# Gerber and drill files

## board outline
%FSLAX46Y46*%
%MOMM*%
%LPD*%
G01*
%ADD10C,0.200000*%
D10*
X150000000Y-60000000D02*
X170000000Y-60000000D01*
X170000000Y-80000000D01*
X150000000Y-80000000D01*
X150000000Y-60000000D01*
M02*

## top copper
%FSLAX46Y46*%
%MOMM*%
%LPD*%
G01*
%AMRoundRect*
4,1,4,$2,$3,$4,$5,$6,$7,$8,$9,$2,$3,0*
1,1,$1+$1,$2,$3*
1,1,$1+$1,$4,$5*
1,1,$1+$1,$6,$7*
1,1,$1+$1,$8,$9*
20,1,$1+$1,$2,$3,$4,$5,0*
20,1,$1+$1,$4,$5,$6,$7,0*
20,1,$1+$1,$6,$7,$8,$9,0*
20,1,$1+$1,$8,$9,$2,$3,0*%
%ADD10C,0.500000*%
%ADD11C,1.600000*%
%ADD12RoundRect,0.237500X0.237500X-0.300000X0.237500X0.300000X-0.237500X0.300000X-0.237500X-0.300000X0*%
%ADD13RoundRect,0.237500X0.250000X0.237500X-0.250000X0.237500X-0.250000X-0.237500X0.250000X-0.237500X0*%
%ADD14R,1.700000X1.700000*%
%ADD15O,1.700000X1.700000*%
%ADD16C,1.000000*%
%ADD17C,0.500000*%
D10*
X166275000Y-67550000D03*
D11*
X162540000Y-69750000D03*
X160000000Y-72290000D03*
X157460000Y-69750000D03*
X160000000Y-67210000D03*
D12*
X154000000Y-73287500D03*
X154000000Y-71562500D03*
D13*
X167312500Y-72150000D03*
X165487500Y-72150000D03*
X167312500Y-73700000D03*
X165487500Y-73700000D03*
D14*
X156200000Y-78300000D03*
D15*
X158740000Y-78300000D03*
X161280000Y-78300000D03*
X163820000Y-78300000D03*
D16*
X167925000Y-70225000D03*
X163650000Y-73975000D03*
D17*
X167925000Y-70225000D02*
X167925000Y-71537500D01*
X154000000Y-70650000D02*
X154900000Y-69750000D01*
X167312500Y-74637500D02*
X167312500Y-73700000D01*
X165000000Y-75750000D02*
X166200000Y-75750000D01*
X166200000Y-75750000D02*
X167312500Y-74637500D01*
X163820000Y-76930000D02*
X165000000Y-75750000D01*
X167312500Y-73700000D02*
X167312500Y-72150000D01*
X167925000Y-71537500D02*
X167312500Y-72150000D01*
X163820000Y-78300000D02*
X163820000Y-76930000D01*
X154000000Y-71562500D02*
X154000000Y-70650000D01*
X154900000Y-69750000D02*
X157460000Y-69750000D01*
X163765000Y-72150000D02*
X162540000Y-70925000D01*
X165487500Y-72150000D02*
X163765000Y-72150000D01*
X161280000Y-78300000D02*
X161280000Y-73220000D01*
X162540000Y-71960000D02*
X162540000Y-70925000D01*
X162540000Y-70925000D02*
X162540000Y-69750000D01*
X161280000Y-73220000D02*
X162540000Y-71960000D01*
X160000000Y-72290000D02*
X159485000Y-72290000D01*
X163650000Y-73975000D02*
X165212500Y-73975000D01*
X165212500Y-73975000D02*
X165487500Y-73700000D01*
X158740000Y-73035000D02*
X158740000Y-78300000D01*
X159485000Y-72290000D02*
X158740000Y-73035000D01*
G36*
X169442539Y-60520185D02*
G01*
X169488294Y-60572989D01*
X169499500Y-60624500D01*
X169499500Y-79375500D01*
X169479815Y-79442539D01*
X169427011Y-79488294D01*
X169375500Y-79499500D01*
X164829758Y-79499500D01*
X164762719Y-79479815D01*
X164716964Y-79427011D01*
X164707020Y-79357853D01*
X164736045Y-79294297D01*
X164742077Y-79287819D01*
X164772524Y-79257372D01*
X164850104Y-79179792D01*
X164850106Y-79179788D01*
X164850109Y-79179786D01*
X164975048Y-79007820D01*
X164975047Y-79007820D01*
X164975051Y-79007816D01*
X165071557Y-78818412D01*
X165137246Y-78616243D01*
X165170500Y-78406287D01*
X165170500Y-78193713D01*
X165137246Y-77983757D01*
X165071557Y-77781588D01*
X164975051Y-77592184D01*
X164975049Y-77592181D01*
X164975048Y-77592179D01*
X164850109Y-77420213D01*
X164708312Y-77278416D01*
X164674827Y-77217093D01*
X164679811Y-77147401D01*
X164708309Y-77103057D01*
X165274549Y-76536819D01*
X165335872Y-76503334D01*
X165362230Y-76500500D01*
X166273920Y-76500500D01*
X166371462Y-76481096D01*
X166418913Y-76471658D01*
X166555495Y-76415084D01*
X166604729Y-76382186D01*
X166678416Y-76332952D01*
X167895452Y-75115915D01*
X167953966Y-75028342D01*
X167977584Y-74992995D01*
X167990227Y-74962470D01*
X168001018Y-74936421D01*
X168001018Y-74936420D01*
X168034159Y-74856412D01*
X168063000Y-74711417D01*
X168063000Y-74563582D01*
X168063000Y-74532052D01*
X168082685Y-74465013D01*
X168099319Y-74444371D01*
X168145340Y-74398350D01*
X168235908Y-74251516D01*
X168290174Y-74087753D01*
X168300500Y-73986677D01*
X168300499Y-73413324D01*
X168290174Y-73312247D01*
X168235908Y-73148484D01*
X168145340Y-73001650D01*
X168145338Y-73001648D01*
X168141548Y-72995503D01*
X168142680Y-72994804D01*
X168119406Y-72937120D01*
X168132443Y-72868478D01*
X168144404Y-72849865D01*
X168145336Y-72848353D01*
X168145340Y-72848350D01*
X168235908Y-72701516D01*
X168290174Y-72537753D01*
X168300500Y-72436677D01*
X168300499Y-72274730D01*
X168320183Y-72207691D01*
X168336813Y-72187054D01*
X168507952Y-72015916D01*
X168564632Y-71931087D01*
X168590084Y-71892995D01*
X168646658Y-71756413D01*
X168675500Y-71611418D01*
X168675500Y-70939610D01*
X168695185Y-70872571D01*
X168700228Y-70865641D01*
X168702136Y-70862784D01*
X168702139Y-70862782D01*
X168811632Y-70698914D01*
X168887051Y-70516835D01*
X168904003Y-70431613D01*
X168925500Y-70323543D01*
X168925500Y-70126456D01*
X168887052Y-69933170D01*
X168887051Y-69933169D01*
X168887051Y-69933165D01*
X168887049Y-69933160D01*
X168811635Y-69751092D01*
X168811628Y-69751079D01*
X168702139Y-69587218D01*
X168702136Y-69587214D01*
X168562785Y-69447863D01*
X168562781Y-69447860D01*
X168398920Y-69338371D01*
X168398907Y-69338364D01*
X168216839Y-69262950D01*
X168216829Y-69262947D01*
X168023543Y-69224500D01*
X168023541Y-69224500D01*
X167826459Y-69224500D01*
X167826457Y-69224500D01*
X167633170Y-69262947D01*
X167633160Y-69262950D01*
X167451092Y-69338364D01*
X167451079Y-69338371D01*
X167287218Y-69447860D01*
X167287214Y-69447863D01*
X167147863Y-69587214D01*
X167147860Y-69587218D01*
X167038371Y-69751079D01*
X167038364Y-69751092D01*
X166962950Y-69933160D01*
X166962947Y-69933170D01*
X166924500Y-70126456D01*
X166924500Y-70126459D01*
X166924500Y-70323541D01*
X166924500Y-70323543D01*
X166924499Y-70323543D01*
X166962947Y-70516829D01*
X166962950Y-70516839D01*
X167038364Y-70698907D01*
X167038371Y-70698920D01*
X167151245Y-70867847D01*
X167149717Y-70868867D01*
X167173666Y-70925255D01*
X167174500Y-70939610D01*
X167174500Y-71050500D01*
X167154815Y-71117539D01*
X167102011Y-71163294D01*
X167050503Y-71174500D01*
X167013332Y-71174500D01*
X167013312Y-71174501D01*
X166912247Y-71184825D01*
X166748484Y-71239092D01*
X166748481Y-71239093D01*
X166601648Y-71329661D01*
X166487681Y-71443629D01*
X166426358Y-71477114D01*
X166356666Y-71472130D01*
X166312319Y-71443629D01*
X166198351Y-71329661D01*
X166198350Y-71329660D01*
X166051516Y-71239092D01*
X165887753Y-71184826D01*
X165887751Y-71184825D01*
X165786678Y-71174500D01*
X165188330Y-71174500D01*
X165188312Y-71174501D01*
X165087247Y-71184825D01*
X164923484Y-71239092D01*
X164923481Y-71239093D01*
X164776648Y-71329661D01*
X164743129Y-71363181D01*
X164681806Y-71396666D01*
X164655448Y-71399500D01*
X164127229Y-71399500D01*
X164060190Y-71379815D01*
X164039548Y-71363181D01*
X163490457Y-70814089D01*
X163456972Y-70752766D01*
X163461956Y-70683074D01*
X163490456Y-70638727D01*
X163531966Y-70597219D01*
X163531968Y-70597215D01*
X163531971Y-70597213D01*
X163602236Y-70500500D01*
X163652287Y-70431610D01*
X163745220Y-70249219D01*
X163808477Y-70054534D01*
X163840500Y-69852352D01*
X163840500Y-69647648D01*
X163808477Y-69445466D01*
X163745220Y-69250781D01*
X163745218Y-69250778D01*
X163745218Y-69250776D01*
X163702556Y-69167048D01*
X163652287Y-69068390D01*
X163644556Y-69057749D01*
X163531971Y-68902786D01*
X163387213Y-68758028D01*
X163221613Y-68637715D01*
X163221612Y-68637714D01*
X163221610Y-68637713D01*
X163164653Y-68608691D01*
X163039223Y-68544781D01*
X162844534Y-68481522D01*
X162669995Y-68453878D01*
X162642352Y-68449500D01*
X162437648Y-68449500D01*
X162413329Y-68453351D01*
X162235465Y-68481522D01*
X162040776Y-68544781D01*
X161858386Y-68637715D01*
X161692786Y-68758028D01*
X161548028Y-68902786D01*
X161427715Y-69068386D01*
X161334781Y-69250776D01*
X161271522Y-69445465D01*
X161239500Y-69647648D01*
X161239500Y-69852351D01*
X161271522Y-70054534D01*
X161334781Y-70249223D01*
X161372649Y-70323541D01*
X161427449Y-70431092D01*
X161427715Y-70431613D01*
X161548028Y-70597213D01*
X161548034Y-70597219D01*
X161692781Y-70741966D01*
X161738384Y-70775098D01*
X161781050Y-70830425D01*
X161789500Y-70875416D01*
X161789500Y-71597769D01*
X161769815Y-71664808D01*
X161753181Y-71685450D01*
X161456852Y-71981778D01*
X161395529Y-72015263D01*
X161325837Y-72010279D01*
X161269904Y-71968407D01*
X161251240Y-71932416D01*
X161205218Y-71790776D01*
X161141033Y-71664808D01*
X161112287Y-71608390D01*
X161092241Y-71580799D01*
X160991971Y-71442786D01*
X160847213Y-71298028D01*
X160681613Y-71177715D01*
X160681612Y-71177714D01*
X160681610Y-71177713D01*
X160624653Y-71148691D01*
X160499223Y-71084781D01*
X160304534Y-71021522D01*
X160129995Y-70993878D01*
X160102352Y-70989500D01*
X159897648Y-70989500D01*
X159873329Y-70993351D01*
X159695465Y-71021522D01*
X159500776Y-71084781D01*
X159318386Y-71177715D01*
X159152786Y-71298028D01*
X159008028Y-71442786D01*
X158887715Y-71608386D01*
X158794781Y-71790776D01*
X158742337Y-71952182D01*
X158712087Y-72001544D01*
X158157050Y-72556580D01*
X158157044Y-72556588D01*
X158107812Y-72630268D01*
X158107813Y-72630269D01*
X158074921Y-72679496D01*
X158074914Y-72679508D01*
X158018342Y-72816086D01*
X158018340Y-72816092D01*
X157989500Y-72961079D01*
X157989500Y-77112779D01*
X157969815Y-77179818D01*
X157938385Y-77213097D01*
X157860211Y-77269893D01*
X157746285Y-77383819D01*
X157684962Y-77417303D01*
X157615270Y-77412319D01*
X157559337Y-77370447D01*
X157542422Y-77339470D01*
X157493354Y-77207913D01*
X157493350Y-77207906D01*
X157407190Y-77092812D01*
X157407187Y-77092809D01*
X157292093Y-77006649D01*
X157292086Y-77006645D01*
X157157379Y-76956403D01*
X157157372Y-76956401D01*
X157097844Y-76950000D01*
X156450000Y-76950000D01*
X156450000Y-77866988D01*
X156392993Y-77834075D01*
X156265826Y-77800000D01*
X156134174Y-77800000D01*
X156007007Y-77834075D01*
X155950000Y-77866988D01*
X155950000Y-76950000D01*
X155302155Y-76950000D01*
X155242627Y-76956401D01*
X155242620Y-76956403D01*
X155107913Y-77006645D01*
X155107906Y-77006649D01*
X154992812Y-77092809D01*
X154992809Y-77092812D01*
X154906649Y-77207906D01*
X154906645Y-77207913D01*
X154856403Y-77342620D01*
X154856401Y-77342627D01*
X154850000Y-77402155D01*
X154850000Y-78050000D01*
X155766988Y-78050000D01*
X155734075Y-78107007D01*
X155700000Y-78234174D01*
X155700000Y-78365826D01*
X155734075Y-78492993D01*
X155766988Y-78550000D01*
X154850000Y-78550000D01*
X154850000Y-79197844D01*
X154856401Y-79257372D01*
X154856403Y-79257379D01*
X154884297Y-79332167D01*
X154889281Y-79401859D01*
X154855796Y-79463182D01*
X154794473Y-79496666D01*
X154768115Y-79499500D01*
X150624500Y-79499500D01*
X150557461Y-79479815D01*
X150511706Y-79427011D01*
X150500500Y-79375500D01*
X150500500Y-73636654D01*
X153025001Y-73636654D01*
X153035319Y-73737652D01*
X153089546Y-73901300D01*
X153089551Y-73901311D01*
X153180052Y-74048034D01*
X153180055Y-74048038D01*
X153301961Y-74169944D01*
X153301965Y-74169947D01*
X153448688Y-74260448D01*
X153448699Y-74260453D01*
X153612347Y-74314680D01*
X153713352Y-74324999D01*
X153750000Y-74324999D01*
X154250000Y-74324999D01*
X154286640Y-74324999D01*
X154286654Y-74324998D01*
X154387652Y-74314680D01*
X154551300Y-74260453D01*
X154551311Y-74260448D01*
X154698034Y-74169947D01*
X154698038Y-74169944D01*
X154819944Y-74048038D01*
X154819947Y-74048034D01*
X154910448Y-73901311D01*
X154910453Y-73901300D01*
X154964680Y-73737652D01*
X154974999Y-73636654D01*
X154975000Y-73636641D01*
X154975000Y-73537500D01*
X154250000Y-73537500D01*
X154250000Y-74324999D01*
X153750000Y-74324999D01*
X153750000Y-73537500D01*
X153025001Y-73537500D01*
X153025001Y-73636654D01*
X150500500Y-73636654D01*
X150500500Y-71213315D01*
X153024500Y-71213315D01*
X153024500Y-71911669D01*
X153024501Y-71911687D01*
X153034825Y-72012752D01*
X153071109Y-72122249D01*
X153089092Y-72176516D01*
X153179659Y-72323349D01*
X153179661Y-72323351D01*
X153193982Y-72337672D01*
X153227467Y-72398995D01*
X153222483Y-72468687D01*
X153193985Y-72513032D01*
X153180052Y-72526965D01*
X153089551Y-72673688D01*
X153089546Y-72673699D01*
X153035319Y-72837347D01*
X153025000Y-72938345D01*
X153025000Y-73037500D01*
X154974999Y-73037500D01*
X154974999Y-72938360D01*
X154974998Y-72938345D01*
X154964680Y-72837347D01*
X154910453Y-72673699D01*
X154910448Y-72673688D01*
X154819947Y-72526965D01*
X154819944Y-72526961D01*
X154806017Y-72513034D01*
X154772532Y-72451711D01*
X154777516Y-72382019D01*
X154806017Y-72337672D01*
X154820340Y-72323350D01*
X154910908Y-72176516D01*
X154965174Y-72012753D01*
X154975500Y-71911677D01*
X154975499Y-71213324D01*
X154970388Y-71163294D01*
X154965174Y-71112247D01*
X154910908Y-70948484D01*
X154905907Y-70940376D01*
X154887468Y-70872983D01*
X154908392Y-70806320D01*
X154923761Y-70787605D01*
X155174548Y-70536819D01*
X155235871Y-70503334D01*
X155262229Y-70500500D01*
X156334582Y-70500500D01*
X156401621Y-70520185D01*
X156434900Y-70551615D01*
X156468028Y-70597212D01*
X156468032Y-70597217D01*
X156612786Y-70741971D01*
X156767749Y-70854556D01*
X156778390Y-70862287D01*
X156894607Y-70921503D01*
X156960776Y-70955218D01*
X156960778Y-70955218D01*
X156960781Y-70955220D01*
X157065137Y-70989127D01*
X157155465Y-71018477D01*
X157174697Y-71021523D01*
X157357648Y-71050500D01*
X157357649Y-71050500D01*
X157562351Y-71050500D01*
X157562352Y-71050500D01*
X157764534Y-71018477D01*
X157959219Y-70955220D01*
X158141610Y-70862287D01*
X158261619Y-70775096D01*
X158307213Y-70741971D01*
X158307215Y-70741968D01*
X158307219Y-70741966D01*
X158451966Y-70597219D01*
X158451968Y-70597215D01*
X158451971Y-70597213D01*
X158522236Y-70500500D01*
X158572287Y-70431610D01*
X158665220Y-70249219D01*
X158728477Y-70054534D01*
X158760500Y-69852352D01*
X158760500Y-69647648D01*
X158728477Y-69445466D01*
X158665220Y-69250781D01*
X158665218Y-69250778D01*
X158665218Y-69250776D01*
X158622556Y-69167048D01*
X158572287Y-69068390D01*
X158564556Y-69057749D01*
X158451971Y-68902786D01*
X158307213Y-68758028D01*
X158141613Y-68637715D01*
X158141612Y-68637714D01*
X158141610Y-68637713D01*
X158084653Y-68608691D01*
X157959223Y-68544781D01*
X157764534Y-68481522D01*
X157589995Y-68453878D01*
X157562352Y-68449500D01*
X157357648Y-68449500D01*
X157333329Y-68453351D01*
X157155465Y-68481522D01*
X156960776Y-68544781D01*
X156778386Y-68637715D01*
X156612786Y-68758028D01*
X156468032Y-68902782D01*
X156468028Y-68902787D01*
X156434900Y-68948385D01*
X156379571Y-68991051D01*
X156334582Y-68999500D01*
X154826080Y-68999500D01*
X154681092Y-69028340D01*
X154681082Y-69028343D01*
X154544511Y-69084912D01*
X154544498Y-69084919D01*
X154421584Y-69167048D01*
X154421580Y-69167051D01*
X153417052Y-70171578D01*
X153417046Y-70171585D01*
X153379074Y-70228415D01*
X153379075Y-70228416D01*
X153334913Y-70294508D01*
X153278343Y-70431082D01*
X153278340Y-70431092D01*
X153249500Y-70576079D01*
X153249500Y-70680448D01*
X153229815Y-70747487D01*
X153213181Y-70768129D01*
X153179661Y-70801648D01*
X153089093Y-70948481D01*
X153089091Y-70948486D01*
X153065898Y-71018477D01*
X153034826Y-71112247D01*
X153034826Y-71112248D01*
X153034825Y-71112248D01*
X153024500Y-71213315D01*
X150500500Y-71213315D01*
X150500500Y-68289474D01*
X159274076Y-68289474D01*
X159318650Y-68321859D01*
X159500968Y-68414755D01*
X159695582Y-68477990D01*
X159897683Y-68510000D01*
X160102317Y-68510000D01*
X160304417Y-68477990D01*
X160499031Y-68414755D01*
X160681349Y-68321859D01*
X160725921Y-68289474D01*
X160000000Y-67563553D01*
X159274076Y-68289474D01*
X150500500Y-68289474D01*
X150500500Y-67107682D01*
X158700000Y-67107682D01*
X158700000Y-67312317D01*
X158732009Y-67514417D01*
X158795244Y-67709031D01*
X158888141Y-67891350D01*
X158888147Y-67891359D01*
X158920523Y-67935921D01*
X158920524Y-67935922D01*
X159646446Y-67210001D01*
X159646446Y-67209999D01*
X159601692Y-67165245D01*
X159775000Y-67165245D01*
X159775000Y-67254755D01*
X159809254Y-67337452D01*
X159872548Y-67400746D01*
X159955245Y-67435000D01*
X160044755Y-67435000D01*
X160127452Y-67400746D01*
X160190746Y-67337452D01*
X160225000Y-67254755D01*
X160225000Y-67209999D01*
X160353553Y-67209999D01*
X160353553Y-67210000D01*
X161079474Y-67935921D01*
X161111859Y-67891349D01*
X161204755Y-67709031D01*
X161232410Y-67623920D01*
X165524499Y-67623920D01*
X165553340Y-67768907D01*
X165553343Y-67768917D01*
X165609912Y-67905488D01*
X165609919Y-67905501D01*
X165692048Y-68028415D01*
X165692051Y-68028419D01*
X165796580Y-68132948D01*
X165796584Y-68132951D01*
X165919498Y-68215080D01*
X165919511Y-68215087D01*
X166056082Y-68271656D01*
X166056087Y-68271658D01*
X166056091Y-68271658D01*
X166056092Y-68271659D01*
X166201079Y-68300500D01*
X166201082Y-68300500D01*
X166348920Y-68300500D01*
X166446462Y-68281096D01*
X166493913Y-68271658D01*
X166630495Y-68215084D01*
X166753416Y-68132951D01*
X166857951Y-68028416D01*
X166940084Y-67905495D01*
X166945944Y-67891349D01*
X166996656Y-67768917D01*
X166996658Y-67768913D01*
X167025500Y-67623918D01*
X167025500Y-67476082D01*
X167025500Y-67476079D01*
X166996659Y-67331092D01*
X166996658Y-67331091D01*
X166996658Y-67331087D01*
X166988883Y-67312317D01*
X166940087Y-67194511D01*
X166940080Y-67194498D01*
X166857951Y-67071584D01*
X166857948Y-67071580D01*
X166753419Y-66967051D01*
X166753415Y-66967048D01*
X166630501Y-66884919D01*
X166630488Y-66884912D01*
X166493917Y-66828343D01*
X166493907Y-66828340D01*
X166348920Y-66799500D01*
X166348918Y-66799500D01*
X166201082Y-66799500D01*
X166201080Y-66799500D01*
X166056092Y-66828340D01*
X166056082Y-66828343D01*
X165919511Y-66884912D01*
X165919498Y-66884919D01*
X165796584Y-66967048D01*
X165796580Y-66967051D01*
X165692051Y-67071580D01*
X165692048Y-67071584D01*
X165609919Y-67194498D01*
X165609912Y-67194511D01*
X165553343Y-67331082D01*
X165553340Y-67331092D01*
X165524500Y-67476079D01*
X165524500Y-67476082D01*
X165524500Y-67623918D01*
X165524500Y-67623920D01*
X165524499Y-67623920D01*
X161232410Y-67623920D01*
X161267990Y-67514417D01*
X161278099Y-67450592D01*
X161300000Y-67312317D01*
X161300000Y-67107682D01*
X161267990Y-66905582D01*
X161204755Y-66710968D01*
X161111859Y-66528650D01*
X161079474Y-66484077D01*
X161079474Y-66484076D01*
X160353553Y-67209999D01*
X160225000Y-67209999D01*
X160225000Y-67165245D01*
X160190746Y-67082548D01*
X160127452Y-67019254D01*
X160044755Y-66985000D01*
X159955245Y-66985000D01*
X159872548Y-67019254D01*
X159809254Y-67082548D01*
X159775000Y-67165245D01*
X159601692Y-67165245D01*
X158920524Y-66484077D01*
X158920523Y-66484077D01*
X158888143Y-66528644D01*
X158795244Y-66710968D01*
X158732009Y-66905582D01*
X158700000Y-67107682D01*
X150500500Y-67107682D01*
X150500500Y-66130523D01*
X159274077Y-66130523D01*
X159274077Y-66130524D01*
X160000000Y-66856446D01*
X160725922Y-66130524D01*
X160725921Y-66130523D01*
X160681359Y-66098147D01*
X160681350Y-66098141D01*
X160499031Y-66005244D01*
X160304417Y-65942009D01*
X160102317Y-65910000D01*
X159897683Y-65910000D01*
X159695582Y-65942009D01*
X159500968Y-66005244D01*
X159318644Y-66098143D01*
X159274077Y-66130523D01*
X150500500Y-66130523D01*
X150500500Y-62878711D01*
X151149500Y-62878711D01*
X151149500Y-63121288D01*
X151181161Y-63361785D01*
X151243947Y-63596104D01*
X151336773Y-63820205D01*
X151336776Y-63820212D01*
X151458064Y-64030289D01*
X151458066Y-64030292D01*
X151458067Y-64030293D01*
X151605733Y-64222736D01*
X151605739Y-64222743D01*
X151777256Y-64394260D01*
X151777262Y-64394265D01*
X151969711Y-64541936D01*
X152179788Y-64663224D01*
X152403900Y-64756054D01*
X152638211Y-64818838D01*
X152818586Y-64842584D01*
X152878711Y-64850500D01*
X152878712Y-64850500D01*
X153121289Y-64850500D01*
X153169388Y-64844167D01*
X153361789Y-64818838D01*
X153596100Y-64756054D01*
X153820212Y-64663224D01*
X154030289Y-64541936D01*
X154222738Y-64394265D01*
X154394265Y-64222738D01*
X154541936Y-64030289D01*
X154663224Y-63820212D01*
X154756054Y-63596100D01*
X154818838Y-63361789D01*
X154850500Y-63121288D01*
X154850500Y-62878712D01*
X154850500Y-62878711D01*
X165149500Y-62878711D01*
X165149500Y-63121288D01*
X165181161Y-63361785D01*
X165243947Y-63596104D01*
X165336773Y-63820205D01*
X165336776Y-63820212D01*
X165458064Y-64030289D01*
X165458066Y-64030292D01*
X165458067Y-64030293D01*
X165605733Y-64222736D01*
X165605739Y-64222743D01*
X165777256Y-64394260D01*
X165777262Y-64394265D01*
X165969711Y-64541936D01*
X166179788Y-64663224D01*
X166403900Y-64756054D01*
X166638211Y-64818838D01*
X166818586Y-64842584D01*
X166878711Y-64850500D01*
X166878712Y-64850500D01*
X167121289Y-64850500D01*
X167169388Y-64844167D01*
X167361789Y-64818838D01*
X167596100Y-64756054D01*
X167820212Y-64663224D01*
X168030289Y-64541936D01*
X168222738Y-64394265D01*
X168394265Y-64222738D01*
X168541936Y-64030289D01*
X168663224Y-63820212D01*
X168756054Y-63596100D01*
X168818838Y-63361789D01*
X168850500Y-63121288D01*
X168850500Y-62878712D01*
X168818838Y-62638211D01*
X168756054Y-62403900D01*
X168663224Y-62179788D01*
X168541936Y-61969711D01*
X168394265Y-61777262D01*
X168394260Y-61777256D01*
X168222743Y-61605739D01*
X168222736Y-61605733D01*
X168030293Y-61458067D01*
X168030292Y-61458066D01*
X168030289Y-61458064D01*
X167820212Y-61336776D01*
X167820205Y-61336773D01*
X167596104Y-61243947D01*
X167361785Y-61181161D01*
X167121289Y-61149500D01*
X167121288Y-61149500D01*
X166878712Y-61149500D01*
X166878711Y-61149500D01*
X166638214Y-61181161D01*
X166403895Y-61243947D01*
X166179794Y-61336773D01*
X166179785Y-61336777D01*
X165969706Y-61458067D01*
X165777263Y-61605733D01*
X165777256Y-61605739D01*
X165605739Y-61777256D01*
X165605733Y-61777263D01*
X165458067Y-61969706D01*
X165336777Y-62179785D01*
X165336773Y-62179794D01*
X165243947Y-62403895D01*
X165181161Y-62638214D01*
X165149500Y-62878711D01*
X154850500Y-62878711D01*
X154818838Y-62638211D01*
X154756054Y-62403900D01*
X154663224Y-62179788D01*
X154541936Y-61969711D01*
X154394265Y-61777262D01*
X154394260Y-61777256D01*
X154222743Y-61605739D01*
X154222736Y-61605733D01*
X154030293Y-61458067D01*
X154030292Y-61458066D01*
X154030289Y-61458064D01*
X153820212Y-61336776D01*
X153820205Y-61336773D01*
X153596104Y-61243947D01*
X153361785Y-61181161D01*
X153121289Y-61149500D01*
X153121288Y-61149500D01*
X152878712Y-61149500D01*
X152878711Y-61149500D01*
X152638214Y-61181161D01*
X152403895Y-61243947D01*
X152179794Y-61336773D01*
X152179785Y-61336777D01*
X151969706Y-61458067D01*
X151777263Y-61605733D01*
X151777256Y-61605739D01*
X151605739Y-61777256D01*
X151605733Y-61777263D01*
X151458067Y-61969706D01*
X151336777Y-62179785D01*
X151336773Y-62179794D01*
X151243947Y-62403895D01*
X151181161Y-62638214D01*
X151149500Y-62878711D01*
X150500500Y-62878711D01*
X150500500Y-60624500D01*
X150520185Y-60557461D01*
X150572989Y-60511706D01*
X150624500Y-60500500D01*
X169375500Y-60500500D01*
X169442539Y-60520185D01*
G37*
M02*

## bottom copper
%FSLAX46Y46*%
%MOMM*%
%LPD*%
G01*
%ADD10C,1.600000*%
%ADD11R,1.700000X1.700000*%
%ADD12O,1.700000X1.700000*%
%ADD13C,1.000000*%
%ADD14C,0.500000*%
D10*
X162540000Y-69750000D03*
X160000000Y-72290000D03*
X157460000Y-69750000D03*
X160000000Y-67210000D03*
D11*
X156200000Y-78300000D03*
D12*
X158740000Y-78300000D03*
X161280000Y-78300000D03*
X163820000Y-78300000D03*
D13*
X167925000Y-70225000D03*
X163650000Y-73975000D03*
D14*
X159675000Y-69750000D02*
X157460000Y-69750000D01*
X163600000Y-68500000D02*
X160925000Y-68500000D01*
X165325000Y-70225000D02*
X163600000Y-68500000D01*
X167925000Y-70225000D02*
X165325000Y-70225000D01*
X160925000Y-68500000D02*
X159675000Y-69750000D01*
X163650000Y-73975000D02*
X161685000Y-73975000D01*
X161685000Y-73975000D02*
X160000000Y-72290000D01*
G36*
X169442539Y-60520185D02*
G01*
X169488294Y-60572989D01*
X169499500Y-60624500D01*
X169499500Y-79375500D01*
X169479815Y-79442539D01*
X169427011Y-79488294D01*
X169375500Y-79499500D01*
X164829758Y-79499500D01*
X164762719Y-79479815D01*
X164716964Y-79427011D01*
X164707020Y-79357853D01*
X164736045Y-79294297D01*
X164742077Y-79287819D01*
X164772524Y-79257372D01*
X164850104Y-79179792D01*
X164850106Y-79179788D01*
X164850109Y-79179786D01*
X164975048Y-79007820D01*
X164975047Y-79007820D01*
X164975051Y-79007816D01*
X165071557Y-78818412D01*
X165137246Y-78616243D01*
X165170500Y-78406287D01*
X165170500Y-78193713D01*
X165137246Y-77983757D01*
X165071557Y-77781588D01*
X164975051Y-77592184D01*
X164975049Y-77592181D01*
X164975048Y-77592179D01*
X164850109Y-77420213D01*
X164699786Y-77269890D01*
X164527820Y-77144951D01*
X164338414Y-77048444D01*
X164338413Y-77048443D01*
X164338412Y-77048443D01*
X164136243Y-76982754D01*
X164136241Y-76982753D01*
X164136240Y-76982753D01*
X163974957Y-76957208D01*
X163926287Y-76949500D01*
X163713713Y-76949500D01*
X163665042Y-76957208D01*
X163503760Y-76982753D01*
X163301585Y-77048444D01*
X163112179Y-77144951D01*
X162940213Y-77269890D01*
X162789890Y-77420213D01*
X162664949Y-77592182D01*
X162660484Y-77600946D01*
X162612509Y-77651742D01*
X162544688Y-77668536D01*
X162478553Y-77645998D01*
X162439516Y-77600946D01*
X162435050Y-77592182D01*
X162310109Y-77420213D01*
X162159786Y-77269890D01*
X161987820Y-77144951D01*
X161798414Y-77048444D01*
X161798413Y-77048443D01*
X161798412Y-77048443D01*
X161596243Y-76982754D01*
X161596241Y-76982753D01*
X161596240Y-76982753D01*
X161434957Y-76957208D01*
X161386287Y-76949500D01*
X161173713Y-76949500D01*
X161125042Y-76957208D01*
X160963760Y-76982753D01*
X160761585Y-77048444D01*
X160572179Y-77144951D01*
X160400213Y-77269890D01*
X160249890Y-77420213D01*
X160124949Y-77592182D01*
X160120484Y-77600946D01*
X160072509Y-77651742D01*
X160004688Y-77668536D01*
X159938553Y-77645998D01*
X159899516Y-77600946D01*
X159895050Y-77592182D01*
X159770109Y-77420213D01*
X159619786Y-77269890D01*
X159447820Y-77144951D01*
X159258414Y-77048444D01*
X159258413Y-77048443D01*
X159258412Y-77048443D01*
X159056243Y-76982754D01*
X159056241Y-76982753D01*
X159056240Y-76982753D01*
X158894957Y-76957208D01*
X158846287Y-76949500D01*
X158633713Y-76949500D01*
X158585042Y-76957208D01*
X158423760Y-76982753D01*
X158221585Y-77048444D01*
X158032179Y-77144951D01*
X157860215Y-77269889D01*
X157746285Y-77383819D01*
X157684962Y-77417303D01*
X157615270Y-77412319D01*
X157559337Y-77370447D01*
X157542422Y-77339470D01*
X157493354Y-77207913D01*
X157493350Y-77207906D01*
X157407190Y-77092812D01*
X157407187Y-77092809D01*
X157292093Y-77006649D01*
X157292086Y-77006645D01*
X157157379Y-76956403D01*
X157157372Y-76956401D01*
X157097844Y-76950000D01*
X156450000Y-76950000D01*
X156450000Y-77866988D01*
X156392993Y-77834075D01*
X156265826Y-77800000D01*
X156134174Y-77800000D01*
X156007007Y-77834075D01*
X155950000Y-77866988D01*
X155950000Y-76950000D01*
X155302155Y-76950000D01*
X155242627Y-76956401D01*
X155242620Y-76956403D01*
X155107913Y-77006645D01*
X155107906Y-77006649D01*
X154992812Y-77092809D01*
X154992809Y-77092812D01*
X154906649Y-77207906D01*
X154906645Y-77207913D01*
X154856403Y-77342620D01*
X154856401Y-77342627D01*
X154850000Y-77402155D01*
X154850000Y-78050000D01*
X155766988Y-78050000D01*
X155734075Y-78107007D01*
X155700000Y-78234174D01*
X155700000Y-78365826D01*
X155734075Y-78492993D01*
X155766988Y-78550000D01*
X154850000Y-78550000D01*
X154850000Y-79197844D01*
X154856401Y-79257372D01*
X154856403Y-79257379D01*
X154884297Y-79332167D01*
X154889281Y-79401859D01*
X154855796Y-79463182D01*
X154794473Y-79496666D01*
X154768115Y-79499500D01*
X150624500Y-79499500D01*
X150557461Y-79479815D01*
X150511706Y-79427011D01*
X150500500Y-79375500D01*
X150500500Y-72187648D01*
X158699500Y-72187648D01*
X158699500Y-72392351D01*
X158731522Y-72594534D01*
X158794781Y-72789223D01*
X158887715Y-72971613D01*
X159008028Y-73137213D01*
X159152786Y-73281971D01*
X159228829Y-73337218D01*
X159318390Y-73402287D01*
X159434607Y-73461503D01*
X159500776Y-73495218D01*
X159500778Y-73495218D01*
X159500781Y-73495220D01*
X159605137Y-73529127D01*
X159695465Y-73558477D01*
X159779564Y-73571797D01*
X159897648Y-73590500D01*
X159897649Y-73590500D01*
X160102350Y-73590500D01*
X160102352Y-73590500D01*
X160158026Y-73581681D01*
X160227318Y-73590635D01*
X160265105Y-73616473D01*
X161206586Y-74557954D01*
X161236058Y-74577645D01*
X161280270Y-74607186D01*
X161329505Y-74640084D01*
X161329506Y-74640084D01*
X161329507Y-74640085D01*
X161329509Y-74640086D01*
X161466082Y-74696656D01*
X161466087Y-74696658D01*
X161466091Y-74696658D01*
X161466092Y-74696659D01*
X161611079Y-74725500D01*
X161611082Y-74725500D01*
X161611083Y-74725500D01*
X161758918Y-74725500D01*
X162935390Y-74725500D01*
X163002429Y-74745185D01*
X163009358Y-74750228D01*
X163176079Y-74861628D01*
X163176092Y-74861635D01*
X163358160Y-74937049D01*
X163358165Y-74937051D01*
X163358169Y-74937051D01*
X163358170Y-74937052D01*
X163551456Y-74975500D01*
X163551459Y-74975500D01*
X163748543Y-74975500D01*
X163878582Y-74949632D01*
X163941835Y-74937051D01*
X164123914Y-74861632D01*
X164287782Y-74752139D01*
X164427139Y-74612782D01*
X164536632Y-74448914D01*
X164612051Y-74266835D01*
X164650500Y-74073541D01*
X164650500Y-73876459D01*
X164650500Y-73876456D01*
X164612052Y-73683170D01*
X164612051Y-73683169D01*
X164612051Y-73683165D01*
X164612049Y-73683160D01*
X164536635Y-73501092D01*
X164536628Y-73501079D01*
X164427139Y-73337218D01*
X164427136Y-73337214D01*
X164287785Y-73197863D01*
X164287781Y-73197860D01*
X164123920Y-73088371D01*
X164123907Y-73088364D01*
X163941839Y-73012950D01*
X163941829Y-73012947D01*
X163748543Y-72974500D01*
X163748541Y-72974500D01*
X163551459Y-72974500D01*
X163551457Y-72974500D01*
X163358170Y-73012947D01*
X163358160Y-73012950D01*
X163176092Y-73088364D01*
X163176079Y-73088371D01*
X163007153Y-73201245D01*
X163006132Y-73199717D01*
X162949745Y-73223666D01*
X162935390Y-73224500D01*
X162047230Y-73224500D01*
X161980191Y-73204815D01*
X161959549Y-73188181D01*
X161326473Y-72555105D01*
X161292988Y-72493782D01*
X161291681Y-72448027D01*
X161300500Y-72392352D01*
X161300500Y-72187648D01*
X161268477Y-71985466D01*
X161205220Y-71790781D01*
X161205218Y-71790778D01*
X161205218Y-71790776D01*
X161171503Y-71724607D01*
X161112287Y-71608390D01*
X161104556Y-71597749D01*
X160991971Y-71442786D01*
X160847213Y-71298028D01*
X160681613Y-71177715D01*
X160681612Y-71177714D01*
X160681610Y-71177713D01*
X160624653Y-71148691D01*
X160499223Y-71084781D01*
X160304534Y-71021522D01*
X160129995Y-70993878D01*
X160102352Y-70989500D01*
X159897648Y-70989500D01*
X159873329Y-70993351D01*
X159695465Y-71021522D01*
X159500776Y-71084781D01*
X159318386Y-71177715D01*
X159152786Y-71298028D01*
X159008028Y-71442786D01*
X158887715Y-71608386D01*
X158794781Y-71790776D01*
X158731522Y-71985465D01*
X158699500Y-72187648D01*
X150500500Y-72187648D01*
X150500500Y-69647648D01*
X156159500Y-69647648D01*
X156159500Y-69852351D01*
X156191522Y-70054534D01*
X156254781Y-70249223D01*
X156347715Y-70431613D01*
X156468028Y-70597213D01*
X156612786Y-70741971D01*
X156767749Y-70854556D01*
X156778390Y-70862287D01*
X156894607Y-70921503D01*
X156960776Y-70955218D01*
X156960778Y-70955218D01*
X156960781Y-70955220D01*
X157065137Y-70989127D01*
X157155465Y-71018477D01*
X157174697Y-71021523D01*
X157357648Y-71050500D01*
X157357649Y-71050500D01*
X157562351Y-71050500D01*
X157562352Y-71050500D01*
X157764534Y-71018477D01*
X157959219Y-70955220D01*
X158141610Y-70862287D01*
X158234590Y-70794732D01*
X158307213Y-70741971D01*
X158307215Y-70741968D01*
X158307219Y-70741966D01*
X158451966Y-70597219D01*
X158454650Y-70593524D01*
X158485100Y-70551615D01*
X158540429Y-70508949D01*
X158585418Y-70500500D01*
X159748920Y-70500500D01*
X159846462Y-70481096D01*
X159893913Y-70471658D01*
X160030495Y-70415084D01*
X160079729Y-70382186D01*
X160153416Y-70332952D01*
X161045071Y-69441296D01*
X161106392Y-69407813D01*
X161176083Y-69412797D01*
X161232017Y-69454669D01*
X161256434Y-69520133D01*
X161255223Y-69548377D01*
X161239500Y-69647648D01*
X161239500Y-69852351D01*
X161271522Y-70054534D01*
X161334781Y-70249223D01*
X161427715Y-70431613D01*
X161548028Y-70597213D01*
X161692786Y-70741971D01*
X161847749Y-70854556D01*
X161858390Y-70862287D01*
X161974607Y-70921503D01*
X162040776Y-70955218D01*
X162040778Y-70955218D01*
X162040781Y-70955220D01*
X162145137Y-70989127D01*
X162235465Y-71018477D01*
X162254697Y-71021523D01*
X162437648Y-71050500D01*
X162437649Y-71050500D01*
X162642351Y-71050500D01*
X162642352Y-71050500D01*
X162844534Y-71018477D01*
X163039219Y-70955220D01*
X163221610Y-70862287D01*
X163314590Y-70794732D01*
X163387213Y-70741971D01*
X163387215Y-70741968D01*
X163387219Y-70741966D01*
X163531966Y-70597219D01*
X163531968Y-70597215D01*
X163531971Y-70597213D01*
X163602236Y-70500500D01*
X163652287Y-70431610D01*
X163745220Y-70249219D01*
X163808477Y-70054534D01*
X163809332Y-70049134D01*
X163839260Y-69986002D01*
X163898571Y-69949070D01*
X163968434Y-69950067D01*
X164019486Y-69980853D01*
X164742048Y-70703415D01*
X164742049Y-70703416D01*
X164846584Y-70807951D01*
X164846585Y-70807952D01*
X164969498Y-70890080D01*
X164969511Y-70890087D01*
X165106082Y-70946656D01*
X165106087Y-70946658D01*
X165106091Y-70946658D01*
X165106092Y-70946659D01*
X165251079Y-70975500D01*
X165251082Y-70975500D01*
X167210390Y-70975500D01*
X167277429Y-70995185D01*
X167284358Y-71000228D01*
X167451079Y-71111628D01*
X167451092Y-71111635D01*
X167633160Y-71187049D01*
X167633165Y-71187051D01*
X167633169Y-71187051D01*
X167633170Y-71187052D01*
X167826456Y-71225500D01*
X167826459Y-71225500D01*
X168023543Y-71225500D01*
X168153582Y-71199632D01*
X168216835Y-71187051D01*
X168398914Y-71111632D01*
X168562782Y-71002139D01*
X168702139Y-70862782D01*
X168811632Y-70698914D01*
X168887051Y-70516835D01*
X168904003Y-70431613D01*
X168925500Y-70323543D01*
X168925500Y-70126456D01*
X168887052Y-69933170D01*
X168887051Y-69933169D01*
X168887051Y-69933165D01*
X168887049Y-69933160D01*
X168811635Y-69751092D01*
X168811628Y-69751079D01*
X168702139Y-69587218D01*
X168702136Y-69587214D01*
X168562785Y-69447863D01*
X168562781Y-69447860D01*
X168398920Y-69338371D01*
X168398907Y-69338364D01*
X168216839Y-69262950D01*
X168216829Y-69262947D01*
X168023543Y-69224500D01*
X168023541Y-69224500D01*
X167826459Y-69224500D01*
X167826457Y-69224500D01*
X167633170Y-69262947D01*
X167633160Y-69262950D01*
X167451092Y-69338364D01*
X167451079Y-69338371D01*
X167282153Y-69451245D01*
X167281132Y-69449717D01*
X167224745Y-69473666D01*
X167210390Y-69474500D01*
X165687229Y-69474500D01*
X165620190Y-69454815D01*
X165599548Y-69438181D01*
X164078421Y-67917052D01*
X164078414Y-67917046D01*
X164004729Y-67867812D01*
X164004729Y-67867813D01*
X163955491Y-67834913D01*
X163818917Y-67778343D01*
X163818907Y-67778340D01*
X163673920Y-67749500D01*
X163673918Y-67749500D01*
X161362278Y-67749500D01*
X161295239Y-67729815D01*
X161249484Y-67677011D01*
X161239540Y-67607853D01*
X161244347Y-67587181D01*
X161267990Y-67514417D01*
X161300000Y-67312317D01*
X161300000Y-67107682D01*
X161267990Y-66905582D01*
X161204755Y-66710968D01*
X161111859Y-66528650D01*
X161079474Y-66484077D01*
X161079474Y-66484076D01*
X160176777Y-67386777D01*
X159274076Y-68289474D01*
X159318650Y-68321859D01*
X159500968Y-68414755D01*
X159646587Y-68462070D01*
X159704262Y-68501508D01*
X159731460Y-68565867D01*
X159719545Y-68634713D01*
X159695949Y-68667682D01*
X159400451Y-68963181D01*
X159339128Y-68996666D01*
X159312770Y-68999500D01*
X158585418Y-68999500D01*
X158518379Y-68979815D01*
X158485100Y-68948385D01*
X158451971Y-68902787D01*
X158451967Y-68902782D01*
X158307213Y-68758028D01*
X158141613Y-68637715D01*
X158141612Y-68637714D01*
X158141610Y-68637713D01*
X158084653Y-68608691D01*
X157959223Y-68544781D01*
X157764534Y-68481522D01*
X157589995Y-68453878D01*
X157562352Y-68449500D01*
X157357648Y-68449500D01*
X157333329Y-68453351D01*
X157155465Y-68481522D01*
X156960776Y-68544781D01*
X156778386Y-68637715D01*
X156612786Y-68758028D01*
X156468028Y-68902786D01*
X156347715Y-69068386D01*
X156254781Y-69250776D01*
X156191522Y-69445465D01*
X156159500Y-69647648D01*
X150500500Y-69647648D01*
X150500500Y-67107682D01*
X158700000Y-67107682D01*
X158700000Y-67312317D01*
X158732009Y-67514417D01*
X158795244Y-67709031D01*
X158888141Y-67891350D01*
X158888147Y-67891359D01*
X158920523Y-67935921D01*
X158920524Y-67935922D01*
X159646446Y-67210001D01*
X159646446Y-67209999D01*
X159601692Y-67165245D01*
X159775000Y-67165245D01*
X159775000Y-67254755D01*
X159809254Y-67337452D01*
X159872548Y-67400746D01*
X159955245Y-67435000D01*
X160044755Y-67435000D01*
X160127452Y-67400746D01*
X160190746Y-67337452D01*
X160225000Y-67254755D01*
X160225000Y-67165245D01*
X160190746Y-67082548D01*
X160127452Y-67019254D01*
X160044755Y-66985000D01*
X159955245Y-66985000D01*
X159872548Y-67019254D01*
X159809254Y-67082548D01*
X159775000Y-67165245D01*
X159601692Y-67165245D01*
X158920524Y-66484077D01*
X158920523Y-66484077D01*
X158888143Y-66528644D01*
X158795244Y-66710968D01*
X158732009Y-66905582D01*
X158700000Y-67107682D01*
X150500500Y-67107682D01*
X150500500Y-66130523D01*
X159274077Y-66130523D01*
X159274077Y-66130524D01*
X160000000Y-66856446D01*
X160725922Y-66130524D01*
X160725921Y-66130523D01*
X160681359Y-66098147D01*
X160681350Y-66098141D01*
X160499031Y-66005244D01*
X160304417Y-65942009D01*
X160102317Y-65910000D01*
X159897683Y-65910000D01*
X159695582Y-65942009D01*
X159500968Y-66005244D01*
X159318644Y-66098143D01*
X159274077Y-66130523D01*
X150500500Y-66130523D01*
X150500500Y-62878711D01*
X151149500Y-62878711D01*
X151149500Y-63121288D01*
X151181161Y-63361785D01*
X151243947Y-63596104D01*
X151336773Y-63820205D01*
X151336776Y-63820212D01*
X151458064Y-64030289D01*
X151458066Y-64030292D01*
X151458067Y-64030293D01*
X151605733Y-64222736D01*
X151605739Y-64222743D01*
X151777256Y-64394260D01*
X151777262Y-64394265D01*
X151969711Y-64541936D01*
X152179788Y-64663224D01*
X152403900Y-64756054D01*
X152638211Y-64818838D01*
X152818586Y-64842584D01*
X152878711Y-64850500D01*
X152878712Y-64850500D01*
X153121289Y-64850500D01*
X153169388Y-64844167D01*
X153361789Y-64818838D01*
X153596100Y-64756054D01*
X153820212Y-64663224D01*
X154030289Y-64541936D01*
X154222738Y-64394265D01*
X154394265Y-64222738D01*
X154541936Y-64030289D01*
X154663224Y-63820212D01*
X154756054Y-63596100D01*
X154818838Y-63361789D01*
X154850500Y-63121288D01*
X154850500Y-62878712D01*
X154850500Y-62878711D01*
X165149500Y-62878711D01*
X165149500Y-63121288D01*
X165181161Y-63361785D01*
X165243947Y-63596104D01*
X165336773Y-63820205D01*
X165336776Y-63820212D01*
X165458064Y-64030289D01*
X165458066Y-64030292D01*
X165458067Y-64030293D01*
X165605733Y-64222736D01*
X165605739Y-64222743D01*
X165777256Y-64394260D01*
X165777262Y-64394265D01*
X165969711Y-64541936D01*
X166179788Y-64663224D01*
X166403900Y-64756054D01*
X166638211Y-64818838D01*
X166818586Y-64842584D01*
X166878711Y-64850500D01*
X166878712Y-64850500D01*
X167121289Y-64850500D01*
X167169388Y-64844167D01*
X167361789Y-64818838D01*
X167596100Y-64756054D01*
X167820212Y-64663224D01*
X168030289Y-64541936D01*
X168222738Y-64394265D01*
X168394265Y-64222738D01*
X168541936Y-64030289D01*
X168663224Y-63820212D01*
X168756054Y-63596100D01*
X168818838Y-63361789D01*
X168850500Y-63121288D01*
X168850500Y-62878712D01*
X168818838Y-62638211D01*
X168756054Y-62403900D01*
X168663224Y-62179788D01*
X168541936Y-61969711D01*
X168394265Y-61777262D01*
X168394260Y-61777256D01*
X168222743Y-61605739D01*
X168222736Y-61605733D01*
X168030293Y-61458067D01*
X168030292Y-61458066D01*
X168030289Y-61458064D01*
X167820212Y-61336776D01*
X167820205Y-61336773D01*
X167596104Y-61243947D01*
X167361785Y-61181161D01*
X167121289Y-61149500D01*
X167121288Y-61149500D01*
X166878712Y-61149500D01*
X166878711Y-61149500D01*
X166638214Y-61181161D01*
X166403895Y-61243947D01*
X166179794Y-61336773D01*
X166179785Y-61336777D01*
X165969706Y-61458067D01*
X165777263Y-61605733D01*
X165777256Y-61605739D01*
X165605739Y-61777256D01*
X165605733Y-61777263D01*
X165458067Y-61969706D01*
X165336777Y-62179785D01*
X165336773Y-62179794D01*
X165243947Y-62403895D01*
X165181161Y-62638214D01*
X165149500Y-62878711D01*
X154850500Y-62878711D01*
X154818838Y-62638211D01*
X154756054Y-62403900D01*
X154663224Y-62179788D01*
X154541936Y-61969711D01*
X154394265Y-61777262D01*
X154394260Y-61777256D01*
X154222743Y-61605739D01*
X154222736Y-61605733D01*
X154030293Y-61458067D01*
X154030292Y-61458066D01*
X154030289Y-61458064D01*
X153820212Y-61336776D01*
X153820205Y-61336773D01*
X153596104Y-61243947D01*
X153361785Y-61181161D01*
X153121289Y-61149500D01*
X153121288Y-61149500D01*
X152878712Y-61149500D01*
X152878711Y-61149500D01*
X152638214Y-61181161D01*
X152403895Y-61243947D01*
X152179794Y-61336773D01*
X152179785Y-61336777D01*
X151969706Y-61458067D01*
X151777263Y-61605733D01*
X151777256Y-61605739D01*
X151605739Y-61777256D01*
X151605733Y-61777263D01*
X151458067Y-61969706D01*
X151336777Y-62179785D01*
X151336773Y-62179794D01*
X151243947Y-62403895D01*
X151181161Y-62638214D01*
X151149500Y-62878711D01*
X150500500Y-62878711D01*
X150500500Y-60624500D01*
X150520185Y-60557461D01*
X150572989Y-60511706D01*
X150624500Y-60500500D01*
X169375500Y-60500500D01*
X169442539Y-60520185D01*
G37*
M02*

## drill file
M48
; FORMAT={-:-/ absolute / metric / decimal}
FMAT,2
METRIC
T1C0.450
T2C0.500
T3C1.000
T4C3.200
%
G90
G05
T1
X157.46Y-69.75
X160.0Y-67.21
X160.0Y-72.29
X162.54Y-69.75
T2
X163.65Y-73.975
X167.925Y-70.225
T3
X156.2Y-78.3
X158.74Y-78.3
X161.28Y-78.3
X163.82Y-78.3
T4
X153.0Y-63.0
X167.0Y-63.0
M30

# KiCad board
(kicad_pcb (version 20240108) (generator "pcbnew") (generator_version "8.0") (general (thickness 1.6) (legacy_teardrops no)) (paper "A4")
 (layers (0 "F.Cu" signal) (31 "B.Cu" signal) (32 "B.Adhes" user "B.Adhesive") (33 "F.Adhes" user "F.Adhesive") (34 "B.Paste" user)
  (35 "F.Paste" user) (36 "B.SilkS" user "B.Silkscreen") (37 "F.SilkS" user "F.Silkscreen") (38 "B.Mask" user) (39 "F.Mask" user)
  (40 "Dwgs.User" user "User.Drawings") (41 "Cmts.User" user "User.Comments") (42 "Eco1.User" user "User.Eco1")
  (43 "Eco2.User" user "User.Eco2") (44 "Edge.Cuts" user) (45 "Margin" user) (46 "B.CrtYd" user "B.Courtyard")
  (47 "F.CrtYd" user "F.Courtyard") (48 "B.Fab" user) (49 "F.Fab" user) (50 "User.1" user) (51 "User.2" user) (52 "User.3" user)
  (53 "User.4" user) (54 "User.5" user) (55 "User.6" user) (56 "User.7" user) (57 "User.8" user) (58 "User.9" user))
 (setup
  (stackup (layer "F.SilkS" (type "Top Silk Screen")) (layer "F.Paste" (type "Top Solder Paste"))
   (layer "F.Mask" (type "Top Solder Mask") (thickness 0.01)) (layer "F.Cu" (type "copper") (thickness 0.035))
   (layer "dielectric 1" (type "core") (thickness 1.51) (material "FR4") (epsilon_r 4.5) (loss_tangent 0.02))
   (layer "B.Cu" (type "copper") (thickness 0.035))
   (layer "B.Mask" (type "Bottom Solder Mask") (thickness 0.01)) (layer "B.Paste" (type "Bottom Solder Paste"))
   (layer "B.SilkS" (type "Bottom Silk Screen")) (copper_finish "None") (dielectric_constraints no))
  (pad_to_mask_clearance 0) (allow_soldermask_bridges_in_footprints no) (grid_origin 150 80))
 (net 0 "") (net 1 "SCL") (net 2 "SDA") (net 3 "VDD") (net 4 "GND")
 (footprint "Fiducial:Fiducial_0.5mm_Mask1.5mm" (layer "F.Cu") (at 166.275 67.55)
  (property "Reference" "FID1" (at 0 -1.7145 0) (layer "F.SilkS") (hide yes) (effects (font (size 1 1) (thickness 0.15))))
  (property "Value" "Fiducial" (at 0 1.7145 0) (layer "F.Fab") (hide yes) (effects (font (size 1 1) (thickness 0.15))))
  (pad "" smd circle (at 0 0) (size 0.5 0.5) (layers "F.Cu" "F.Mask") (solder_mask_margin 0.5) (clearance 0.5)))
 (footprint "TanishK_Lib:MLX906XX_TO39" (layer "F.Cu") (at 160 69.75 -90)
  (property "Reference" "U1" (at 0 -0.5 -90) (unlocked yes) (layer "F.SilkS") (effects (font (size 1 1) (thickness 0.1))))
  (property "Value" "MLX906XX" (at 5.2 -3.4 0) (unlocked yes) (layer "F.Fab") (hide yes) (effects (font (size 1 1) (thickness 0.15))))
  (pad "1" thru_hole circle (at 0 -2.54 270) (size 1.6 1.6) (drill 0.45) (layers "*.Cu" "*.Mask") (remove_unused_layers no) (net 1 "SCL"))
  (pad "2" thru_hole circle (at 2.54 0 270) (size 1.6 1.6) (drill 0.45) (layers "*.Cu" "*.Mask") (remove_unused_layers no) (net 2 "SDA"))
  (pad "3" thru_hole circle (at 0 2.54 270) (size 1.6 1.6) (drill 0.45) (layers "*.Cu" "*.Mask") (remove_unused_layers no) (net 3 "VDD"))
  (pad "4" thru_hole circle (at -2.54 0 270) (size 1.6 1.6) (drill 0.45) (layers "*.Cu" "*.Mask") (remove_unused_layers no) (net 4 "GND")))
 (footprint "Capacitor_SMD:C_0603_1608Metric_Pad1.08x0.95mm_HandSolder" (layer "F.Cu") (at 154 72.425 90)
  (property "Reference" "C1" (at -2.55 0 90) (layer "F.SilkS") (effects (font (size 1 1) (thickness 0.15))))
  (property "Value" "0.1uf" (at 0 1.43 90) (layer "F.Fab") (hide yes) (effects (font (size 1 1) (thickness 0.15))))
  (pad "1" smd roundrect (at -0.8625 0 90) (size 1.075 0.95) (layers "F.Cu" "F.Paste" "F.Mask") (roundrect_rratio 0.25) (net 4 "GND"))
  (pad "2" smd roundrect (at 0.8625 0 90) (size 1.075 0.95) (layers "F.Cu" "F.Paste" "F.Mask") (roundrect_rratio 0.25) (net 3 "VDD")))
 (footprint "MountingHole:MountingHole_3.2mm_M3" (layer "F.Cu") (at 153 63)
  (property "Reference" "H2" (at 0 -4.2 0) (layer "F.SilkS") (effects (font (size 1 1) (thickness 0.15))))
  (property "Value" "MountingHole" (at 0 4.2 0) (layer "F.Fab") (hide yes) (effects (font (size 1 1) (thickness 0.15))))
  (pad "" np_thru_hole circle (at 0 0) (size 3.2 3.2) (drill 3.2) (layers "*.Cu" "*.Mask")))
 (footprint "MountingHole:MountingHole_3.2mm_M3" (layer "F.Cu") (at 167 63)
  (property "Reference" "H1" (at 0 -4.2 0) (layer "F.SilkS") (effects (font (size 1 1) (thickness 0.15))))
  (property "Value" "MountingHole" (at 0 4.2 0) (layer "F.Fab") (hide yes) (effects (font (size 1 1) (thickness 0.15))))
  (pad "" np_thru_hole circle (at 0 0) (size 3.2 3.2) (drill 3.2) (layers "*.Cu" "*.Mask")))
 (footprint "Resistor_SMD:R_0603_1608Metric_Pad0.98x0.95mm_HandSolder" (layer "F.Cu") (at 166.4 72.15 180)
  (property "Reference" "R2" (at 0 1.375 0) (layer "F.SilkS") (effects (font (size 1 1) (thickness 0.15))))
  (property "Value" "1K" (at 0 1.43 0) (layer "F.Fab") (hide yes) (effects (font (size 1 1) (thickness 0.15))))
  (pad "1" smd roundrect (at -0.9125 0 180) (size 0.975 0.95) (layers "F.Cu" "F.Paste" "F.Mask") (roundrect_rratio 0.25) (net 3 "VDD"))
  (pad "2" smd roundrect (at 0.9125 0 180) (size 0.975 0.95) (layers "F.Cu" "F.Paste" "F.Mask") (roundrect_rratio 0.25) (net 1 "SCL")))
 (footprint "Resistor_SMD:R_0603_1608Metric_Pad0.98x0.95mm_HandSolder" (layer "F.Cu") (at 166.4 73.7 180)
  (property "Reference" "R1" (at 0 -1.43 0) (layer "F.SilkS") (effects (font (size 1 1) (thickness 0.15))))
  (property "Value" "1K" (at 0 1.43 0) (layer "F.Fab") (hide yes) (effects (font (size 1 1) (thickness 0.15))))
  (pad "1" smd roundrect (at -0.9125 0 180) (size 0.975 0.95) (layers "F.Cu" "F.Paste" "F.Mask") (roundrect_rratio 0.25) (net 3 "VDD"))
  (pad "2" smd roundrect (at 0.9125 0 180) (size 0.975 0.95) (layers "F.Cu" "F.Paste" "F.Mask") (roundrect_rratio 0.25) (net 2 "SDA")))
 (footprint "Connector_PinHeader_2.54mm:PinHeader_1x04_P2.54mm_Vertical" (layer "F.Cu") (at 156.2 78.3 90)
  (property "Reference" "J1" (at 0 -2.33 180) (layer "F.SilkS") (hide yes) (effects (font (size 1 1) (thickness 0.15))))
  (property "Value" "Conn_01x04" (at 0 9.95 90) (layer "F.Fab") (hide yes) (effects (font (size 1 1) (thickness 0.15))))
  (pad "1" thru_hole rect (at 0 0 90) (size 1.7 1.7) (drill 1) (layers "*.Cu" "*.Mask") (remove_unused_layers no) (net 4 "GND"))
  (pad "2" thru_hole oval (at 0 2.54 90) (size 1.7 1.7) (drill 1) (layers "*.Cu" "*.Mask") (remove_unused_layers no) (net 2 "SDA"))
  (pad "3" thru_hole oval (at 0 5.08 90) (size 1.7 1.7) (drill 1) (layers "*.Cu" "*.Mask") (remove_unused_layers no) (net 1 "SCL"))
  (pad "4" thru_hole oval (at 0 7.62 90) (size 1.7 1.7) (drill 1) (layers "*.Cu" "*.Mask") (remove_unused_layers no) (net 3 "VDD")))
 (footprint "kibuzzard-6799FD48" (layer "F.Cu") (at 156.15 75.696338 90)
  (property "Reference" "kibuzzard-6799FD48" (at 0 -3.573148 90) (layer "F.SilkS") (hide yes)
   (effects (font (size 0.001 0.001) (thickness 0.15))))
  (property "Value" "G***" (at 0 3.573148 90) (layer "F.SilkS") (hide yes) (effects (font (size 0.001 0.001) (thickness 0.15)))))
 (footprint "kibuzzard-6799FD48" (layer "B.Cu") (at 156.15 75.7 -90)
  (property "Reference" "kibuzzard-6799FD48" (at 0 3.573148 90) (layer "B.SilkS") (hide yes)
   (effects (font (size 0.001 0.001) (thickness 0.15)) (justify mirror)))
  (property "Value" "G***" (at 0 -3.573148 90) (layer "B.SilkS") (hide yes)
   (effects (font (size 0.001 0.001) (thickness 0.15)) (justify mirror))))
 (gr_rect (start 150 60) (end 170 80) (stroke (width 0.2) (type default)) (fill none) (layer "Edge.Cuts"))
 (segment (start 167.925 70.225) (end 167.925 71.5375) (width 0.5) (layer "F.Cu") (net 3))
 (segment (start 154 70.65) (end 154.9 69.75) (width 0.5) (layer "F.Cu") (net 3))
 (segment (start 167.3125 74.6375) (end 167.3125 73.7) (width 0.5) (layer "F.Cu") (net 3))
 (segment (start 165 75.75) (end 166.2 75.75) (width 0.5) (layer "F.Cu") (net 3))
 (segment (start 166.2 75.75) (end 167.3125 74.6375) (width 0.5) (layer "F.Cu") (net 3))
 (segment (start 163.82 76.93) (end 165 75.75) (width 0.5) (layer "F.Cu") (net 3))
 (segment (start 167.3125 73.7) (end 167.3125 72.15) (width 0.5) (layer "F.Cu") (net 3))
 (segment (start 167.925 71.5375) (end 167.3125 72.15) (width 0.5) (layer "F.Cu") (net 3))
 (segment (start 163.82 78.3) (end 163.82 76.93) (width 0.5) (layer "F.Cu") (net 3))
 (segment (start 154 71.5625) (end 154 70.65) (width 0.5) (layer "F.Cu") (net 3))
 (segment (start 154.9 69.75) (end 157.46 69.75) (width 0.5) (layer "F.Cu") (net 3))
 (via (at 167.925 70.225) (size 1) (drill 0.5) (layers "F.Cu" "B.Cu") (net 3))
 (segment (start 159.675 69.75) (end 157.46 69.75) (width 0.5) (layer "B.Cu") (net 3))
 (segment (start 163.6 68.5) (end 160.925 68.5) (width 0.5) (layer "B.Cu") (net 3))
 (segment (start 165.325 70.225) (end 163.6 68.5) (width 0.5) (layer "B.Cu") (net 3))
 (segment (start 167.925 70.225) (end 165.325 70.225) (width 0.5) (layer "B.Cu") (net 3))
 (segment (start 160.925 68.5) (end 159.675 69.75) (width 0.5) (layer "B.Cu") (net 3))
 (segment (start 163.765 72.15) (end 162.54 70.925) (width 0.5) (layer "F.Cu") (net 1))
 (segment (start 165.4875 72.15) (end 163.765 72.15) (width 0.5) (layer "F.Cu") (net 1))
 (segment (start 161.28 78.3) (end 161.28 73.22) (width 0.5) (layer "F.Cu") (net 1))
 (segment (start 162.54 71.96) (end 162.54 70.925) (width 0.5) (layer "F.Cu") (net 1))
 (segment (start 162.54 70.925) (end 162.54 69.75) (width 0.5) (layer "F.Cu") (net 1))
 (segment (start 161.28 73.22) (end 162.54 71.96) (width 0.5) (layer "F.Cu") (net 1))
 (segment (start 160 72.29) (end 159.485 72.29) (width 0.5) (layer "F.Cu") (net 2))
 (segment (start 163.65 73.975) (end 165.2125 73.975) (width 0.5) (layer "F.Cu") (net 2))
 (segment (start 165.2125 73.975) (end 165.4875 73.7) (width 0.5) (layer "F.Cu") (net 2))
 (segment (start 158.74 73.035) (end 158.74 78.3) (width 0.5) (layer "F.Cu") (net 2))
 (segment (start 159.485 72.29) (end 158.74 73.035) (width 0.5) (layer "F.Cu") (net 2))
 (via (at 163.65 73.975) (size 1) (drill 0.5) (layers "F.Cu" "B.Cu") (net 2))
 (segment (start 163.65 73.975) (end 161.685 73.975) (width 0.5) (layer "B.Cu") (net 2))
 (segment (start 161.685 73.975) (end 160 72.29) (width 0.5) (layer "B.Cu") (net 2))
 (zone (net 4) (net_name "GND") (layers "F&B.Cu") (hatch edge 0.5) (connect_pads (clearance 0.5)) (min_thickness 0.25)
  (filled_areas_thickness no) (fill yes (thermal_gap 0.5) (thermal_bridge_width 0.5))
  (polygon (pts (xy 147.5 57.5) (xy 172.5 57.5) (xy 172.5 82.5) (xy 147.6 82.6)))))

